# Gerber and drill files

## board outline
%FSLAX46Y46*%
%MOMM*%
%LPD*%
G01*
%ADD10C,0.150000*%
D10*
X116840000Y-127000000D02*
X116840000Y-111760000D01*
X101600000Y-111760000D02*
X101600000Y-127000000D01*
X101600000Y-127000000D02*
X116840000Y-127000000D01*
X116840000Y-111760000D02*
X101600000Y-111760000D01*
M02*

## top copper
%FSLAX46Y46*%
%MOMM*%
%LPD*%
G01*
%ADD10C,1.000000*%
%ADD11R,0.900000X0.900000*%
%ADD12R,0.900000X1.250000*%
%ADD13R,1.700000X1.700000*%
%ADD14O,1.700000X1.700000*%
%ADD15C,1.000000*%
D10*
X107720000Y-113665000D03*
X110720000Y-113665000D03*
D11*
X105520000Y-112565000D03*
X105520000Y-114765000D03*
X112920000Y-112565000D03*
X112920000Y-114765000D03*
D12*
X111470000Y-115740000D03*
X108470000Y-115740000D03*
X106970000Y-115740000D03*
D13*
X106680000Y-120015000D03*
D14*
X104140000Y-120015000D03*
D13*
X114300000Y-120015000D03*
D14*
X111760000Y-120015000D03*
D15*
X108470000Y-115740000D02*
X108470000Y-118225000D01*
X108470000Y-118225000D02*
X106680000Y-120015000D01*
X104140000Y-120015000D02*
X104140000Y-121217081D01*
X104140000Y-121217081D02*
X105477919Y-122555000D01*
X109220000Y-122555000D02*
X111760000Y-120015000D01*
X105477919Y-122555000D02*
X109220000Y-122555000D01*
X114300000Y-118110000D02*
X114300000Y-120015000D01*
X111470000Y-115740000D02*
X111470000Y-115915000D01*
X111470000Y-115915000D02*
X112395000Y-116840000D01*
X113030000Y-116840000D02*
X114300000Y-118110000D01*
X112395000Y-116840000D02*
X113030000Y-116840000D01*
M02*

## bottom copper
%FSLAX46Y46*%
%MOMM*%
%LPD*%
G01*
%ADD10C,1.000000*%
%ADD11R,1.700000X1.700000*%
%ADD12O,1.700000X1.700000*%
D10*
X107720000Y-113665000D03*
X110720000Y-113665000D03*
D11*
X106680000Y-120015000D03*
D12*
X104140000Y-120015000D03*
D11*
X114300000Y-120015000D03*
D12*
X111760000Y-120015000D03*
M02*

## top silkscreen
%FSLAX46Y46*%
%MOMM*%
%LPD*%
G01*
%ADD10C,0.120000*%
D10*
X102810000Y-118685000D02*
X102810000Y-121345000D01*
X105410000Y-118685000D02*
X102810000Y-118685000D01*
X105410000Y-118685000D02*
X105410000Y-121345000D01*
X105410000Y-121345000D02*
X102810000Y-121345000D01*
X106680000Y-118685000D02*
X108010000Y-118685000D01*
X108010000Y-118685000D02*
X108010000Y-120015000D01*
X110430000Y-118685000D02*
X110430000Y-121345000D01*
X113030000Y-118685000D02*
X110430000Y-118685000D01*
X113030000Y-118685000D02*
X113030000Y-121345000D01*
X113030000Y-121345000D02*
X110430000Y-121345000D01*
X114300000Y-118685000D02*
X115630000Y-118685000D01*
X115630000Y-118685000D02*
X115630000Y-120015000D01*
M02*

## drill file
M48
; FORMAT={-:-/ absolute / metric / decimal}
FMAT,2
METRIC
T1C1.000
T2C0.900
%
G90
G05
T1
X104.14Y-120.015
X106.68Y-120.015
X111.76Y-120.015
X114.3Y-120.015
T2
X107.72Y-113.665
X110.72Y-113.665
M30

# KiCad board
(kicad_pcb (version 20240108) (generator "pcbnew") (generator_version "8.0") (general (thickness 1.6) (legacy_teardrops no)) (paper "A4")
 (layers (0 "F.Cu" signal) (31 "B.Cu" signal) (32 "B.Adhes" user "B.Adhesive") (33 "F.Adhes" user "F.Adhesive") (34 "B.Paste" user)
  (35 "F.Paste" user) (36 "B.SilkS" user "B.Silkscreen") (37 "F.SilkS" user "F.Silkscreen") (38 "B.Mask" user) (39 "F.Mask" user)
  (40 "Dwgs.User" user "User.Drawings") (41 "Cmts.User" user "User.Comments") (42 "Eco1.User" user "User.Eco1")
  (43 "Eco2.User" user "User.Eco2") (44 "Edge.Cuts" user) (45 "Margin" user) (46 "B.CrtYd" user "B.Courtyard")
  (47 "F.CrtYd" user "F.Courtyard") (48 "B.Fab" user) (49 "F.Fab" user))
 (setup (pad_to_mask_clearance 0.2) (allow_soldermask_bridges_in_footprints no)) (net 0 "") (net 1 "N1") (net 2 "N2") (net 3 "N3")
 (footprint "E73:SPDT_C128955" (layer "F.Cu") (at 109.22 113.665)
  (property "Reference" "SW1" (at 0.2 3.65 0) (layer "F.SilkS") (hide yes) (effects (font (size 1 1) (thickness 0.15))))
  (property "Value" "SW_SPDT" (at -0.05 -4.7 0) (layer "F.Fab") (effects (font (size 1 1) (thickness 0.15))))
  (pad "" np_thru_hole circle (at -1.5 0) (size 1 1) (drill 0.9) (layers "*.Cu" "*.Mask"))
  (pad "" np_thru_hole circle (at 1.5 0) (size 1 1) (drill 0.9) (layers "*.Cu" "*.Mask"))
  (pad "0" smd rect (at -3.7 -1.1) (size 0.9 0.9) (layers "F.Cu" "F.Paste" "F.Mask"))
  (pad "0" smd rect (at -3.7 1.1) (size 0.9 0.9) (layers "F.Cu" "F.Paste" "F.Mask"))
  (pad "0" smd rect (at 3.7 -1.1) (size 0.9 0.9) (layers "F.Cu" "F.Paste" "F.Mask"))
  (pad "0" smd rect (at 3.7 1.1) (size 0.9 0.9) (layers "F.Cu" "F.Paste" "F.Mask"))
  (pad "1" smd rect (at 2.25 2.075) (size 0.9 1.25) (layers "F.Cu" "F.Paste" "F.Mask") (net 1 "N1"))
  (pad "2" smd rect (at -0.75 2.075) (size 0.9 1.25) (layers "F.Cu" "F.Paste" "F.Mask") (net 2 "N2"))
  (pad "3" smd rect (at -2.25 2.075) (size 0.9 1.25) (layers "F.Cu" "F.Paste" "F.Mask")))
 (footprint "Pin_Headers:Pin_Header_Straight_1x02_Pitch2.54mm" (layer "F.Cu") (at 106.68 120.015 -90)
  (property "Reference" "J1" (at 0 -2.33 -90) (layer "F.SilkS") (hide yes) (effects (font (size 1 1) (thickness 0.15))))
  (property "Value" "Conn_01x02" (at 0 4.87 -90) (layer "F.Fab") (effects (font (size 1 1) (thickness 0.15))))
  (fp_line (start -1.33 3.87) (end 1.33 3.87) (stroke (width 0.12) (type solid)) (layer "F.SilkS"))
  (fp_line (start -1.33 1.27) (end -1.33 3.87) (stroke (width 0.12) (type solid)) (layer "F.SilkS"))
  (fp_line (start -1.33 1.27) (end 1.33 1.27) (stroke (width 0.12) (type solid)) (layer "F.SilkS"))
  (fp_line (start 1.33 1.27) (end 1.33 3.87) (stroke (width 0.12) (type solid)) (layer "F.SilkS"))
  (fp_line (start -1.33 0) (end -1.33 -1.33) (stroke (width 0.12) (type solid)) (layer "F.SilkS"))
  (fp_line (start -1.33 -1.33) (end 0 -1.33) (stroke (width 0.12) (type solid)) (layer "F.SilkS"))
  (pad "1" thru_hole rect (at 0 0 270) (size 1.7 1.7) (drill 1) (layers "*.Cu" "*.Mask") (remove_unused_layers no) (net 2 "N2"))
  (pad "2" thru_hole oval (at 0 2.54 270) (size 1.7 1.7) (drill 1) (layers "*.Cu" "*.Mask") (remove_unused_layers no) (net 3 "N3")))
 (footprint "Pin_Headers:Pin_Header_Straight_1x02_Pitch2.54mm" (layer "F.Cu") (at 114.3 120.015 -90)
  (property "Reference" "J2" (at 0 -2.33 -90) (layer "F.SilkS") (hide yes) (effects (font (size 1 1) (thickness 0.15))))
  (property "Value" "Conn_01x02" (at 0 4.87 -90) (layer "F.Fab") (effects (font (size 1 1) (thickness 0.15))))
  (fp_line (start -1.33 3.87) (end 1.33 3.87) (stroke (width 0.12) (type solid)) (layer "F.SilkS"))
  (fp_line (start -1.33 1.27) (end -1.33 3.87) (stroke (width 0.12) (type solid)) (layer "F.SilkS"))
  (fp_line (start -1.33 1.27) (end 1.33 1.27) (stroke (width 0.12) (type solid)) (layer "F.SilkS"))
  (fp_line (start 1.33 1.27) (end 1.33 3.87) (stroke (width 0.12) (type solid)) (layer "F.SilkS"))
  (fp_line (start -1.33 0) (end -1.33 -1.33) (stroke (width 0.12) (type solid)) (layer "F.SilkS"))
  (fp_line (start -1.33 -1.33) (end 0 -1.33) (stroke (width 0.12) (type solid)) (layer "F.SilkS"))
  (pad "1" thru_hole rect (at 0 0 270) (size 1.7 1.7) (drill 1) (layers "*.Cu" "*.Mask") (remove_unused_layers no) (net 1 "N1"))
  (pad "2" thru_hole oval (at 0 2.54 270) (size 1.7 1.7) (drill 1) (layers "*.Cu" "*.Mask") (remove_unused_layers no) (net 3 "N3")))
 (gr_line (start 116.84 127) (end 116.84 111.76) (stroke (width 0.15) (type solid)) (layer "Edge.Cuts"))
 (gr_line (start 101.6 111.76) (end 101.6 127) (stroke (width 0.15) (type solid)) (layer "Edge.Cuts"))
 (gr_line (start 101.6 127) (end 116.84 127) (stroke (width 0.15) (type solid)) (layer "Edge.Cuts"))
 (gr_line (start 116.84 111.76) (end 101.6 111.76) (stroke (width 0.15) (type solid)) (layer "Edge.Cuts"))
 (segment (start 108.47 115.74) (end 108.47 118.225) (width 1) (layer "F.Cu") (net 2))
 (segment (start 108.47 118.225) (end 106.68 120.015) (width 1) (layer "F.Cu") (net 2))
 (segment (start 104.14 120.015) (end 104.14 121.217081) (width 1) (layer "F.Cu") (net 3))
 (segment (start 104.14 121.217081) (end 105.477919 122.555) (width 1) (layer "F.Cu") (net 3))
 (segment (start 109.22 122.555) (end 111.76 120.015) (width 1) (layer "F.Cu") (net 3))
 (segment (start 105.477919 122.555) (end 109.22 122.555) (width 1) (layer "F.Cu") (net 3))
 (segment (start 114.3 118.11) (end 114.3 120.015) (width 1) (layer "F.Cu") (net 1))
 (segment (start 111.47 115.74) (end 111.47 115.915) (width 1) (layer "F.Cu") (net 1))
 (segment (start 111.47 115.915) (end 112.395 116.84) (width 1) (layer "F.Cu") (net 1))
 (segment (start 113.03 116.84) (end 114.3 118.11) (width 1) (layer "F.Cu") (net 1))
 (segment (start 112.395 116.84) (end 113.03 116.84) (width 1) (layer "F.Cu") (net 1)))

